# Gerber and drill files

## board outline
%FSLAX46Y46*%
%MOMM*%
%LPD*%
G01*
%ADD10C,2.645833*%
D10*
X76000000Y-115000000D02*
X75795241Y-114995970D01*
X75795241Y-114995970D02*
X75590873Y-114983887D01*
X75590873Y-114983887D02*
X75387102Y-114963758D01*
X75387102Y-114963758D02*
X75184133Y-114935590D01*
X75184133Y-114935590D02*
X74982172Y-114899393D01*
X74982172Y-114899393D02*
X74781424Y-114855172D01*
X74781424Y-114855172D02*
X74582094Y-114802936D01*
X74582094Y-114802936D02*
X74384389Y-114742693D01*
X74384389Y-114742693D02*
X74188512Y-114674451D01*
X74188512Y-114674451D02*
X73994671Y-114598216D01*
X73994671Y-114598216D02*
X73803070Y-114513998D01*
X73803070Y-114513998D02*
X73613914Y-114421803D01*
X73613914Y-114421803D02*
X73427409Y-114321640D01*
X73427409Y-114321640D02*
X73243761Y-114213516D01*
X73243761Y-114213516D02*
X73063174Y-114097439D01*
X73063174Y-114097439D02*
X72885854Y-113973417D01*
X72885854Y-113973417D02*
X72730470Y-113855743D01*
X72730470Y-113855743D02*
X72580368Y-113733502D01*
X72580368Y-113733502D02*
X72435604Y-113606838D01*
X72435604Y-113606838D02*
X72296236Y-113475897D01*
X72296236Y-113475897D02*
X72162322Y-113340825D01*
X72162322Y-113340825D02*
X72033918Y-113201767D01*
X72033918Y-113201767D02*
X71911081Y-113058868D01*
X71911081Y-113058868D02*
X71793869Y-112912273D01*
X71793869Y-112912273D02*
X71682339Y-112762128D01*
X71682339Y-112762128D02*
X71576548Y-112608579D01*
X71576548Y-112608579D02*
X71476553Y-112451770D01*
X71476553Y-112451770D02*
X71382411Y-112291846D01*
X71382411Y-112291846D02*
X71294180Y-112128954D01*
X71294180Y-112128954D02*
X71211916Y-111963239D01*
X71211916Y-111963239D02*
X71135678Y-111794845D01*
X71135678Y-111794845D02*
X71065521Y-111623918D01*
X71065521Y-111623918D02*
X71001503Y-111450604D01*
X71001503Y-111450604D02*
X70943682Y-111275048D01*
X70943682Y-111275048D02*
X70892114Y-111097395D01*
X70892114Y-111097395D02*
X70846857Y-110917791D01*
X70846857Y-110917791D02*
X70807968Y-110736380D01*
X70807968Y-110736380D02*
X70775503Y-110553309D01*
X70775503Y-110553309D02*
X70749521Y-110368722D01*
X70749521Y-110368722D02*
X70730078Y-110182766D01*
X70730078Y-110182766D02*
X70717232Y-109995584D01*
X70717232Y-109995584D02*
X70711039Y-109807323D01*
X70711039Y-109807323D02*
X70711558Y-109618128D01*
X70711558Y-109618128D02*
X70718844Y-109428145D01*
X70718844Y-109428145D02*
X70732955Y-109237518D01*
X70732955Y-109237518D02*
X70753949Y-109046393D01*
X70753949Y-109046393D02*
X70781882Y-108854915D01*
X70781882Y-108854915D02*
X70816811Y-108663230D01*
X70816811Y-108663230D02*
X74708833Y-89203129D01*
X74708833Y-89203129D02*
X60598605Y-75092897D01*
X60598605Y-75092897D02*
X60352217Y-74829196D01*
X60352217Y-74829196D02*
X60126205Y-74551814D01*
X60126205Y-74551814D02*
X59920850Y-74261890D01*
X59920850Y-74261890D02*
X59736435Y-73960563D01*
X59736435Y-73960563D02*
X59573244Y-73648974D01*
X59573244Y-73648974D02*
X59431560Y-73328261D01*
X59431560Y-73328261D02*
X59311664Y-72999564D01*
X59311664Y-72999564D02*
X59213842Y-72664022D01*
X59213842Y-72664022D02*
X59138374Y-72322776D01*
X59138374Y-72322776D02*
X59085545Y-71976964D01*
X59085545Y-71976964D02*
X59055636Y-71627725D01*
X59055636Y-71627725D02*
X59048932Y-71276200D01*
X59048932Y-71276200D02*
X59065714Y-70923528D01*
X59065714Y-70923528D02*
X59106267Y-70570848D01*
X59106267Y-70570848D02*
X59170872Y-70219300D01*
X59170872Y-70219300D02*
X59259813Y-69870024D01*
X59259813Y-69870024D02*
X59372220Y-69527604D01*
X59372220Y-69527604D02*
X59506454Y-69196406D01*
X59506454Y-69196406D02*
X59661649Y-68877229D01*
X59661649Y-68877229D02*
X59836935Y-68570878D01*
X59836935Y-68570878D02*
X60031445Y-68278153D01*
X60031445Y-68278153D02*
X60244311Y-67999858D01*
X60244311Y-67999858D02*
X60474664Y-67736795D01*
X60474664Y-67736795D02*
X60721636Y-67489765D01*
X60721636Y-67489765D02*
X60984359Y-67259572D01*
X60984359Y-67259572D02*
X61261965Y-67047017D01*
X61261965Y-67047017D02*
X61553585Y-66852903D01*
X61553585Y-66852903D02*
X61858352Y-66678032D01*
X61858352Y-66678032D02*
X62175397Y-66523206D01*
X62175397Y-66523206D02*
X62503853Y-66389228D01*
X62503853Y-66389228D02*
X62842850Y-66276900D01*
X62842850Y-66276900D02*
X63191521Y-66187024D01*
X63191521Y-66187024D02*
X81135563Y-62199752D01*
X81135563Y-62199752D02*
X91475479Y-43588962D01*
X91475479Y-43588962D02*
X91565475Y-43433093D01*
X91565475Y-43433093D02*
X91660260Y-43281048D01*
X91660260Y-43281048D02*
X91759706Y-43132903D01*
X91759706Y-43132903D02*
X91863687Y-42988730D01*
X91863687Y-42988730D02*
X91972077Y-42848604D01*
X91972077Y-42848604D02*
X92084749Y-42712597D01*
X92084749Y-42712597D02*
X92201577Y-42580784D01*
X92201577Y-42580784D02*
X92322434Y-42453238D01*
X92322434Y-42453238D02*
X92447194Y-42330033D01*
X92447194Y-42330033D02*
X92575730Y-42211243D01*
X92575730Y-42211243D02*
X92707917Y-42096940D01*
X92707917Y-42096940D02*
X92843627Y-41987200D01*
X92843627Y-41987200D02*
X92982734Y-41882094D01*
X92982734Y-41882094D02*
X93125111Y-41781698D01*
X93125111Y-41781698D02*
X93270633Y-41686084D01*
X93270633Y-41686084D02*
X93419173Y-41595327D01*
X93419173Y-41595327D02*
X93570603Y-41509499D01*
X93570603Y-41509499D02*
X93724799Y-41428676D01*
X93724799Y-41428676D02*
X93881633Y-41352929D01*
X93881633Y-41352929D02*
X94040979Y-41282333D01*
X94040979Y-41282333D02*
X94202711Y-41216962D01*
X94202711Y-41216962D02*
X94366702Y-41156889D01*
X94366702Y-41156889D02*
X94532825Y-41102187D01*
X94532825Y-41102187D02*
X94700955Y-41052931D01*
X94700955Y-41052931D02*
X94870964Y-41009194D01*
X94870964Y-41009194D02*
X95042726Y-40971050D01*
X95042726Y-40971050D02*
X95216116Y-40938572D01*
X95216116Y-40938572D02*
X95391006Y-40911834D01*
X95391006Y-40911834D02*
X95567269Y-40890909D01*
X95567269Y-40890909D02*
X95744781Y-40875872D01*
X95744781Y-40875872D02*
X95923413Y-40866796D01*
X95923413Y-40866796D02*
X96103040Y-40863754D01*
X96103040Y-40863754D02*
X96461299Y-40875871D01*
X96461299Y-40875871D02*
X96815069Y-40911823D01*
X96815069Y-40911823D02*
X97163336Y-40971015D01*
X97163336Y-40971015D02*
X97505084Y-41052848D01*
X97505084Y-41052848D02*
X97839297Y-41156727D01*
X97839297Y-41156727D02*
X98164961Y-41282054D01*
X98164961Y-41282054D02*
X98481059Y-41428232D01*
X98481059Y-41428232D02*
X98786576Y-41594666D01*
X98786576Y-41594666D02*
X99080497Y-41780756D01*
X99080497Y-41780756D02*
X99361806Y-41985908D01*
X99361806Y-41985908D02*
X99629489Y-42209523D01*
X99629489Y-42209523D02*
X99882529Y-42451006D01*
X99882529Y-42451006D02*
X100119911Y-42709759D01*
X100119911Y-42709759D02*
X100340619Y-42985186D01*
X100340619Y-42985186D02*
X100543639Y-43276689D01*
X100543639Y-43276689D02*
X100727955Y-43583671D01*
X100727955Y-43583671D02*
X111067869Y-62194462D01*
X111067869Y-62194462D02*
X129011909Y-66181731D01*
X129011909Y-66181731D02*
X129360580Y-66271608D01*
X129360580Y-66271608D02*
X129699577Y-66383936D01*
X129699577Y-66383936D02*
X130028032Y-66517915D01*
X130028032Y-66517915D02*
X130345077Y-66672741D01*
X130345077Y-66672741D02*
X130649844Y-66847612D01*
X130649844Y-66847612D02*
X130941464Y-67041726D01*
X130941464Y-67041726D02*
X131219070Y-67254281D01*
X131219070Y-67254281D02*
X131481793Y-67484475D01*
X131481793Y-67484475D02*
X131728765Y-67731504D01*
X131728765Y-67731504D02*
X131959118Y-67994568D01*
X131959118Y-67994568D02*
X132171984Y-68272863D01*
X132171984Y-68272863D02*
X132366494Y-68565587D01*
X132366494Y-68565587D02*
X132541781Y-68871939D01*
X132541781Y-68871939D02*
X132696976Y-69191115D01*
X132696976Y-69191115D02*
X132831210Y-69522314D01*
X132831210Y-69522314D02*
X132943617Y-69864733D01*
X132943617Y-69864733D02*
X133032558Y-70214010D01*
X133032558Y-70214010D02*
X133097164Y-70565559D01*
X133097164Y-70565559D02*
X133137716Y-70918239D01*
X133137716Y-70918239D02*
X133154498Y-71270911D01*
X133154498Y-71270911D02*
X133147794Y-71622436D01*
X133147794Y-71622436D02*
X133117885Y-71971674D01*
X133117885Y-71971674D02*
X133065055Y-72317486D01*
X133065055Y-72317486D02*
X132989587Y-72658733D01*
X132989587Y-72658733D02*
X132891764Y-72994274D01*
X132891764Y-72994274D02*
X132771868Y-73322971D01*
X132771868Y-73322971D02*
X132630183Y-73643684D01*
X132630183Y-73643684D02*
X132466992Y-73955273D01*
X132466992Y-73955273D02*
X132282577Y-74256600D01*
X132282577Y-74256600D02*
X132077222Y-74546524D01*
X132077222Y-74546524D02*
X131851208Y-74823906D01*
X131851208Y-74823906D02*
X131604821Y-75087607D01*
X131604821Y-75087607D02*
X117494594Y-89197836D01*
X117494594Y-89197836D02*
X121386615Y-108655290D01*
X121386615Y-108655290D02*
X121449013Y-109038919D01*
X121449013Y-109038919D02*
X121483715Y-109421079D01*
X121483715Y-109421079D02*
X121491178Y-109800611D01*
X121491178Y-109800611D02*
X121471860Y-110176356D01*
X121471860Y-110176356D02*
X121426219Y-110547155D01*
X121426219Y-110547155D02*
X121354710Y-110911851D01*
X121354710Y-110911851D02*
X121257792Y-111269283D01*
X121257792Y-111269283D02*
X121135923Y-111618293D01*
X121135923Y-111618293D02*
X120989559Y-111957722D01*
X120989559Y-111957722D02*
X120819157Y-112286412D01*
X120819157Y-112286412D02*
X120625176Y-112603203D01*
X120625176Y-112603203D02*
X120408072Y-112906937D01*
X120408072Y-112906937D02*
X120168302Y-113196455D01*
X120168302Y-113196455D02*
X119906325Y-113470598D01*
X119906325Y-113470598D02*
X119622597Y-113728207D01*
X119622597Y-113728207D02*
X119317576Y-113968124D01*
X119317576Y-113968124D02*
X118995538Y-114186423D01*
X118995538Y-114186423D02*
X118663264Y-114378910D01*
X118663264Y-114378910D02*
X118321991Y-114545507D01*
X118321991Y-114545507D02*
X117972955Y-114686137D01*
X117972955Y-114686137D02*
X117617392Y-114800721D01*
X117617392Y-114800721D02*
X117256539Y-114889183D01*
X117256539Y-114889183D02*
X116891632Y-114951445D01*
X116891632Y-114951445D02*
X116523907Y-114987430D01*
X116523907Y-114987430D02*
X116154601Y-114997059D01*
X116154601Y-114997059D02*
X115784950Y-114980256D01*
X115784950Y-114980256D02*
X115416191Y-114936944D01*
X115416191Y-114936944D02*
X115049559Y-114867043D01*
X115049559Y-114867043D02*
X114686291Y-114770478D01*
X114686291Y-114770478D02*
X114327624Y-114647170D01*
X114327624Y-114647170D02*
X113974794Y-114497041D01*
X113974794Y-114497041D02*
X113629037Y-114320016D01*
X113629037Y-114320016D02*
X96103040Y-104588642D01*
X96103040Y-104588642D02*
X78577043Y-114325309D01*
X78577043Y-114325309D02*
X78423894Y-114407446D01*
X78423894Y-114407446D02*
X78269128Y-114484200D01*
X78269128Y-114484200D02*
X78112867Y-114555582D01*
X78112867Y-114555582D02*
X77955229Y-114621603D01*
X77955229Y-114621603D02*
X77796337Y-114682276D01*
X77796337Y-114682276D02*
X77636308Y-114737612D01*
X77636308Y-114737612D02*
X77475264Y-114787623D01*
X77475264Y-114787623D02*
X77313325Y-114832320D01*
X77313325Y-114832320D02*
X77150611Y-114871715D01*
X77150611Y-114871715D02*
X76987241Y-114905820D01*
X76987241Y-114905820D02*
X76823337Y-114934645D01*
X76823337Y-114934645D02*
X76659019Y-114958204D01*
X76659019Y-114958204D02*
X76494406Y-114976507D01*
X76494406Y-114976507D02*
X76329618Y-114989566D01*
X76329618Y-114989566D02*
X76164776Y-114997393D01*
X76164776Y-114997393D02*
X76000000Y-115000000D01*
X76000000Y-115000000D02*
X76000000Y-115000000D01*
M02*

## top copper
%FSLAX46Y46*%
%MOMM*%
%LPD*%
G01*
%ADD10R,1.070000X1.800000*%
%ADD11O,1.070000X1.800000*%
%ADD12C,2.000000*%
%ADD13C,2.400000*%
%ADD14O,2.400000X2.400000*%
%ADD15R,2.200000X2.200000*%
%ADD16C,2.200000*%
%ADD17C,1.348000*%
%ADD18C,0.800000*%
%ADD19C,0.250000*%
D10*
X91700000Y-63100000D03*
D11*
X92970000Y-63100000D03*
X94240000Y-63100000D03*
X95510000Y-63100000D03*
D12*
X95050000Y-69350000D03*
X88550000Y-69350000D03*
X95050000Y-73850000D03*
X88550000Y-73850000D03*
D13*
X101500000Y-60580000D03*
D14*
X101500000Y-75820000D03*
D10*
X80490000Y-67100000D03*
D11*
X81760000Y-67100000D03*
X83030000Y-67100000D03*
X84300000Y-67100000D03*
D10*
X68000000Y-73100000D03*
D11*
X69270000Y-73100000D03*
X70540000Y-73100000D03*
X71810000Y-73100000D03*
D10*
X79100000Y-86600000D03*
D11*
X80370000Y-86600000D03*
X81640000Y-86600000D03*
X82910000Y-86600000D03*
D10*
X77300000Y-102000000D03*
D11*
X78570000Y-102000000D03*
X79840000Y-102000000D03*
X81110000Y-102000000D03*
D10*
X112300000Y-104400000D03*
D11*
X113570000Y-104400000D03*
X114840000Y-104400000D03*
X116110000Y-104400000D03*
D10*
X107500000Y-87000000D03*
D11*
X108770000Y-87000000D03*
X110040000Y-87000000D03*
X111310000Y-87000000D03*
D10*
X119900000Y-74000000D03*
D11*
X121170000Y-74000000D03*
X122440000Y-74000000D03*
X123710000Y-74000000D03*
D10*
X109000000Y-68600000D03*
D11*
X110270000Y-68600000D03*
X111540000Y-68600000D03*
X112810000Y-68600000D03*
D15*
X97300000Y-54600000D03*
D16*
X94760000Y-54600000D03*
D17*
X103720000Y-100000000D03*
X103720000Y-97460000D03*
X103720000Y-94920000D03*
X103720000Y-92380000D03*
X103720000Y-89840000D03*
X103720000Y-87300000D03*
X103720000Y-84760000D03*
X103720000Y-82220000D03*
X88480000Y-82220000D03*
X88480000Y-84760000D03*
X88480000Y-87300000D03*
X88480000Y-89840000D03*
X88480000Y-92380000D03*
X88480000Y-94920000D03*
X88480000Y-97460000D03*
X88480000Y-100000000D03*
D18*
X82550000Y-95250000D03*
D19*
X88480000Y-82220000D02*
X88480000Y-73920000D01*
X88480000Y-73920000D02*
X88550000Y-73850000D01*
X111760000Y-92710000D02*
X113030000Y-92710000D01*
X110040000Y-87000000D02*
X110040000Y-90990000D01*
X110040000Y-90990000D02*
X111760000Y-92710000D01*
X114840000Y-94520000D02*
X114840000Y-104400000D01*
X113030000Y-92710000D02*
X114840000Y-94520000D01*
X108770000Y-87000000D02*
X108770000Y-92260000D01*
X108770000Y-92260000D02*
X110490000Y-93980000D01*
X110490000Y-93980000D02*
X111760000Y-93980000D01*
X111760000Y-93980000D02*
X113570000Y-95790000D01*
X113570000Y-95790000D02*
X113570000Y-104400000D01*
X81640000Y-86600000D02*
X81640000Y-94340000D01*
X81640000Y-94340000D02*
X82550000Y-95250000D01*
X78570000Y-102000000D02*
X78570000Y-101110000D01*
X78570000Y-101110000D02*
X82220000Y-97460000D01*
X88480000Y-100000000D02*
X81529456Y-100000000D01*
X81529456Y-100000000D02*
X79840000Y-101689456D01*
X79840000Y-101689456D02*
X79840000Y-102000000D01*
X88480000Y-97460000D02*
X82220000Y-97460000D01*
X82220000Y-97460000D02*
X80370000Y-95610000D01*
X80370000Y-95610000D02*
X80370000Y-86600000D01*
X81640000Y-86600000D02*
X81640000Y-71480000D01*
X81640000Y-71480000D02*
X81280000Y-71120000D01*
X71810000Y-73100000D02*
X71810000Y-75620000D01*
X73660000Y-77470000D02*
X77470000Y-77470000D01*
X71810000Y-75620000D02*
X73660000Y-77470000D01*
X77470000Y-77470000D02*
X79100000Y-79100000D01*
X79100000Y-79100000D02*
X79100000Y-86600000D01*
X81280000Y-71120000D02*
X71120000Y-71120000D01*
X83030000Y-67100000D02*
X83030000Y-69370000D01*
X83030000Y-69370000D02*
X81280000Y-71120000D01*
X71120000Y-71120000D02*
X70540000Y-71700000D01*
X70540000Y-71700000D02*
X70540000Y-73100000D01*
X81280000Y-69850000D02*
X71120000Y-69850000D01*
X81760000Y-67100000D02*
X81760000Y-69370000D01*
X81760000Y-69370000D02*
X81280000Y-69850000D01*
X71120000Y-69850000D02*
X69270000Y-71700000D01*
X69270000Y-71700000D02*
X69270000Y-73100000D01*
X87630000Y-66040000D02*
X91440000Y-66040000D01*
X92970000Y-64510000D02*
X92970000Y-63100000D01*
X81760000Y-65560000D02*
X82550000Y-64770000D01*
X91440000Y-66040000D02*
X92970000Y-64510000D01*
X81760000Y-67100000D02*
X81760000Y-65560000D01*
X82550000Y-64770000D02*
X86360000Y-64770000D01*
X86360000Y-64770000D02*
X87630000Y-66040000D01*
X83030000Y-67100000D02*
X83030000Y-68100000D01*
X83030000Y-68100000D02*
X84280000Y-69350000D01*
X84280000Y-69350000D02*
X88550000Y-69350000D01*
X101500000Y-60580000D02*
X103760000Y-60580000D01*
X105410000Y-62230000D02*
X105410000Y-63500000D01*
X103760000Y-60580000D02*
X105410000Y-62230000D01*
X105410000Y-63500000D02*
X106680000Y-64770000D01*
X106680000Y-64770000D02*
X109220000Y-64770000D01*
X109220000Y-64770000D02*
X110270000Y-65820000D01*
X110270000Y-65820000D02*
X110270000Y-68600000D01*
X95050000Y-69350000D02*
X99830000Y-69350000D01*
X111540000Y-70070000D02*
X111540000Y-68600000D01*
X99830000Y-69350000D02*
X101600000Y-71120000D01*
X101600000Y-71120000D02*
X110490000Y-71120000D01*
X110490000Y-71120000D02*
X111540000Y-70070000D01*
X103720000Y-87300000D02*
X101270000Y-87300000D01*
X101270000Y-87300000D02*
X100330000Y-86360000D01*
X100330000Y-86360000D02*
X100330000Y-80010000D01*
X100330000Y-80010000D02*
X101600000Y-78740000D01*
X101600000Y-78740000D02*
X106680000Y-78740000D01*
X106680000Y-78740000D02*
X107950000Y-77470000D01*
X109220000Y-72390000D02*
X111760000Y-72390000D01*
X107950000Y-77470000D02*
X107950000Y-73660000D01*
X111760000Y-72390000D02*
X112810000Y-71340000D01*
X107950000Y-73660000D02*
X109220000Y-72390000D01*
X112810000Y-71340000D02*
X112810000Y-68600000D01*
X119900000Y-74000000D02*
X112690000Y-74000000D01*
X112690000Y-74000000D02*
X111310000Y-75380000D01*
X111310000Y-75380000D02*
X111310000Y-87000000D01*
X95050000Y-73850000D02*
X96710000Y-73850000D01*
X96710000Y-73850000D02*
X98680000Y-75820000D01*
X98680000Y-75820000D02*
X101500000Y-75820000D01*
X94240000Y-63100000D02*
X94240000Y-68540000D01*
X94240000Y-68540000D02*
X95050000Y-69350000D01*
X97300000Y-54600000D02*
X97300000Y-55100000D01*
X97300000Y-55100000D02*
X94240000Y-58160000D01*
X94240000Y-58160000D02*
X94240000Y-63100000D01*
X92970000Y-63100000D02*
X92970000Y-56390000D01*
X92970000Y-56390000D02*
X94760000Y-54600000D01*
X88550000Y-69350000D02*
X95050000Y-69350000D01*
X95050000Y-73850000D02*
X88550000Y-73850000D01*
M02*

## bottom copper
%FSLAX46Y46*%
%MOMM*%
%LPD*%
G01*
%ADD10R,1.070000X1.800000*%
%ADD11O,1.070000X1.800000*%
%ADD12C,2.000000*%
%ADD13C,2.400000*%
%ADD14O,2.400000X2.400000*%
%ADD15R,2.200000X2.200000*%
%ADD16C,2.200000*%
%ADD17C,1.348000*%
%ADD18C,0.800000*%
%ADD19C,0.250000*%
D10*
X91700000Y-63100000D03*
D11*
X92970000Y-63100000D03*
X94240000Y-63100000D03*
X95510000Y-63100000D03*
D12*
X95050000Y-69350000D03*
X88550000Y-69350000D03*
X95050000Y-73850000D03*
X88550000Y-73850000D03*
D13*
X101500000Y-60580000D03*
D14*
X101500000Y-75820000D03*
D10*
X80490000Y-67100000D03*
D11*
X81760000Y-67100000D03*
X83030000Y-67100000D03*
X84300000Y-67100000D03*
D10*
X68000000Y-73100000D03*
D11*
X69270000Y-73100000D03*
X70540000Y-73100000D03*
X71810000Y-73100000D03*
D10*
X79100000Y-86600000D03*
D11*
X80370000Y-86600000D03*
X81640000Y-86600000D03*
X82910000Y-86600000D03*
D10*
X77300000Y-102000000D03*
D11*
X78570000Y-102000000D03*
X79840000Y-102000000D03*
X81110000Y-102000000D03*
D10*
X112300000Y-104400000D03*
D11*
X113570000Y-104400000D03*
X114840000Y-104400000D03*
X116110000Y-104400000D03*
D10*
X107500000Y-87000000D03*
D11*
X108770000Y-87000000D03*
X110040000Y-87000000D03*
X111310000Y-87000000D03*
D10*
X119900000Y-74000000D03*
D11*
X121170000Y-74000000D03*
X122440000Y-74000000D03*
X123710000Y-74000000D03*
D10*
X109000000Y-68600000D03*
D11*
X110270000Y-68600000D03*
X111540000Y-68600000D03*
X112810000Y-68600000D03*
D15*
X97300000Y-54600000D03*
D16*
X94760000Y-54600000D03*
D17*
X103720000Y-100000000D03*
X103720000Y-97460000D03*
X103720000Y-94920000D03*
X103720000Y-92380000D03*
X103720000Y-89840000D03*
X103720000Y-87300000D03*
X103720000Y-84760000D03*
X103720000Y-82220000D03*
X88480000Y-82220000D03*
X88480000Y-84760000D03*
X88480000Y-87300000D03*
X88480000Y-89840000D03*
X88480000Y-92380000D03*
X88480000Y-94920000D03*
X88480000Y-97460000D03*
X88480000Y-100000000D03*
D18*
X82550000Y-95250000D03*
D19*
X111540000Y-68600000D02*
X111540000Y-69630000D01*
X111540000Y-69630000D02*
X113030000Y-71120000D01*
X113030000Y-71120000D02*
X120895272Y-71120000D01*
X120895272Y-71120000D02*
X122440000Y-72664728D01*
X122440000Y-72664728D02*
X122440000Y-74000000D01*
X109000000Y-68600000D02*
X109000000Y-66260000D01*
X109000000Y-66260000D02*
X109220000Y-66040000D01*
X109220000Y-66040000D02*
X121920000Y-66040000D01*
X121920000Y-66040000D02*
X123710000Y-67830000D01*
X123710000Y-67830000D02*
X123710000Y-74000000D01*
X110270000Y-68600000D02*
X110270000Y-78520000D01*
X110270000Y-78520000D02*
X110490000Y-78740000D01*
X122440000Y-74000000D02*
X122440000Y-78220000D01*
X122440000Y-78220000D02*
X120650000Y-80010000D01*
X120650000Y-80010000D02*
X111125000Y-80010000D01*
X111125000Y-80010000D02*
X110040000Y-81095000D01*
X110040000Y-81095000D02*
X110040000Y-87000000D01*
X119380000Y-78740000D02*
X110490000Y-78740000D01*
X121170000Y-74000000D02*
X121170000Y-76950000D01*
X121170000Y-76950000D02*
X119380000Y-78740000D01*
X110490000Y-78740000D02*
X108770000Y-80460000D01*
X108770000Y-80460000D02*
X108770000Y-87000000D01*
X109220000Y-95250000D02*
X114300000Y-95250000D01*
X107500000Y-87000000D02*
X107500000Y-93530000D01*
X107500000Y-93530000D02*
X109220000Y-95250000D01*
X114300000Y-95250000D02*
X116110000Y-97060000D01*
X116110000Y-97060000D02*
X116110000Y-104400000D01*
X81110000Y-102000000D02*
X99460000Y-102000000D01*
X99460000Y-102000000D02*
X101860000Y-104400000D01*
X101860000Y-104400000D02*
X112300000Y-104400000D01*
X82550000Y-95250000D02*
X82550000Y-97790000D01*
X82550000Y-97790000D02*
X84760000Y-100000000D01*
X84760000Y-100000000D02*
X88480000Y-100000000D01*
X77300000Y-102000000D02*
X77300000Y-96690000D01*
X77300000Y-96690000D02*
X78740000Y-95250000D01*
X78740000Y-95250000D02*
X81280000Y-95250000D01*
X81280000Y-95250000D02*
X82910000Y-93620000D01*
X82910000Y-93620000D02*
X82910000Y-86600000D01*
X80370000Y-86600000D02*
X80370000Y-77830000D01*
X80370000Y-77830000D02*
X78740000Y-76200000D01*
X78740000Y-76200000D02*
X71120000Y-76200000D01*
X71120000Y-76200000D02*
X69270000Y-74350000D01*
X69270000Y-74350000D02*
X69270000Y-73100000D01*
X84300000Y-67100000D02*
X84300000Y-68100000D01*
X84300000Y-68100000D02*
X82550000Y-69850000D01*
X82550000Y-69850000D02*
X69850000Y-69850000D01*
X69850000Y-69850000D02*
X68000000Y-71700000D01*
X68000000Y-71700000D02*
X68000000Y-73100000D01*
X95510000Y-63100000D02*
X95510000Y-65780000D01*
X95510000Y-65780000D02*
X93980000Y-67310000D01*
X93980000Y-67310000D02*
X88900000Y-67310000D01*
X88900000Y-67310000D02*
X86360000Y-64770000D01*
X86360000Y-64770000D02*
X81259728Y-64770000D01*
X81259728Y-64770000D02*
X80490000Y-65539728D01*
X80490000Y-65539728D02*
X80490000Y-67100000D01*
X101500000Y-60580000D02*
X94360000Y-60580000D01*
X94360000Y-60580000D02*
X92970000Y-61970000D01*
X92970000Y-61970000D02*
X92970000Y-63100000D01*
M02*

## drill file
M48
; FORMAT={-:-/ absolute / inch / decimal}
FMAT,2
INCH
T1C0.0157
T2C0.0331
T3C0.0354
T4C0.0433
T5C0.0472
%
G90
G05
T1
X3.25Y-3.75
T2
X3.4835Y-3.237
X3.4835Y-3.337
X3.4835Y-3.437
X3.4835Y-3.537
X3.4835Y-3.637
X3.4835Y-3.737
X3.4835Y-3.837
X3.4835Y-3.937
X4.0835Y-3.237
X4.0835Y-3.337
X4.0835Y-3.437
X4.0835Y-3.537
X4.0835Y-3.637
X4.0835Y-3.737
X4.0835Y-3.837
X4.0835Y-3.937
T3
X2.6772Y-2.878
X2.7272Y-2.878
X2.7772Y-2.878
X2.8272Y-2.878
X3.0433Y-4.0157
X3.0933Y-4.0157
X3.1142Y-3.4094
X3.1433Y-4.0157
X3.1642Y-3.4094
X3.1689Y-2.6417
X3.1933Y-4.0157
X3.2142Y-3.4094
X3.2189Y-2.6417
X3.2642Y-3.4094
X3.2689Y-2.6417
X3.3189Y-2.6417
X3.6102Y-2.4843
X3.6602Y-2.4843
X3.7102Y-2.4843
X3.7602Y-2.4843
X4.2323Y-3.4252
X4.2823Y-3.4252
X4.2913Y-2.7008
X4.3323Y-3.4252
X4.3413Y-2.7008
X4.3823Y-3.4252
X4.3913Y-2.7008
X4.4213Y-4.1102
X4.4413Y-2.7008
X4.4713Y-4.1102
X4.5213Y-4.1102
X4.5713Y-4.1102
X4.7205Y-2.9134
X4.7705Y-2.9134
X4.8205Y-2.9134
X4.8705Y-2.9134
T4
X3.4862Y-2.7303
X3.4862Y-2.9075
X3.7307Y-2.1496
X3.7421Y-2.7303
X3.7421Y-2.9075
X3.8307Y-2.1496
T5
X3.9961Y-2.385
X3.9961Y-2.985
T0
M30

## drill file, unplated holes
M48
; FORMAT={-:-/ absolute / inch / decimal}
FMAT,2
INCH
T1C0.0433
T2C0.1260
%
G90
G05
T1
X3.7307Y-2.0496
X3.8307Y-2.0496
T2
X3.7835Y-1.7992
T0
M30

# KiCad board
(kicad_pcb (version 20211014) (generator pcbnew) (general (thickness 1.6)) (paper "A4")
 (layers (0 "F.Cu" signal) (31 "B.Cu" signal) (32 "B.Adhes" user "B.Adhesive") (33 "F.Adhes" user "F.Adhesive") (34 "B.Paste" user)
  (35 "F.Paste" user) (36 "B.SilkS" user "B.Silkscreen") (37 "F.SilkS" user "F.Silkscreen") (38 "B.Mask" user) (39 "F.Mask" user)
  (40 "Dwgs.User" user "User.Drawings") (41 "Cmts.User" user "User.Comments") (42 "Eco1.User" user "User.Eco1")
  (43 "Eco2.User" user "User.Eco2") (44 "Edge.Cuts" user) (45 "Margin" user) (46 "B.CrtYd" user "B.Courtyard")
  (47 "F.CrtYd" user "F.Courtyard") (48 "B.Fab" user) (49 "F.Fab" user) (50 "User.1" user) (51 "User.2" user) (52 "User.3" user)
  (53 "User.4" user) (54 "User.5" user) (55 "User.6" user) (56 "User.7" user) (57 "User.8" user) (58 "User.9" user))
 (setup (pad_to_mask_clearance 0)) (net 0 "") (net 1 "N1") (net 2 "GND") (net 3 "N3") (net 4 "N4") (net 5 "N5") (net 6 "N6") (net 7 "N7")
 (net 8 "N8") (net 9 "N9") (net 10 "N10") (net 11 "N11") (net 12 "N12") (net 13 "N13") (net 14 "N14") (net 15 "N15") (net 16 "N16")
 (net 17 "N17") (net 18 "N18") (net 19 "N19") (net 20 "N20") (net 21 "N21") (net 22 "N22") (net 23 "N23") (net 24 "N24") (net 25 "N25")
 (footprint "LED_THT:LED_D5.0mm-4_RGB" (layer "F.Cu") (at 77.3 102)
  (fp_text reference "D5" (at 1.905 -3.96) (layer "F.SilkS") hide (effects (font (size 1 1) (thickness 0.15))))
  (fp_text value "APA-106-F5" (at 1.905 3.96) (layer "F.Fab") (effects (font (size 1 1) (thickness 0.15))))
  (pad "1" thru_hole rect (at 0 0) (size 1.07 1.8) (drill 0.9) (layers *.Cu *.Mask) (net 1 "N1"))
  (pad "2" thru_hole oval (at 1.27 0) (size 1.07 1.8) (drill 0.9) (layers *.Cu *.Mask) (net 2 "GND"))
  (pad "3" thru_hole oval (at 2.54 0) (size 1.07 1.8) (drill 0.9) (layers *.Cu *.Mask) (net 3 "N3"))
  (pad "4" thru_hole oval (at 3.81 0) (size 1.07 1.8) (drill 0.9) (layers *.Cu *.Mask) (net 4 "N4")))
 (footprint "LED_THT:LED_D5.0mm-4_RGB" (layer "F.Cu") (at 119.9 74)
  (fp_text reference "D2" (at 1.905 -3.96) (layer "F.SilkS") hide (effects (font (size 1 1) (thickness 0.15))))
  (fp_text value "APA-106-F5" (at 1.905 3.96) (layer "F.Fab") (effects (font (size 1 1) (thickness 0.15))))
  (pad "1" thru_hole rect (at 0 0) (size 1.07 1.8) (drill 0.9) (layers *.Cu *.Mask) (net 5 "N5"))
  (pad "2" thru_hole oval (at 1.27 0) (size 1.07 1.8) (drill 0.9) (layers *.Cu *.Mask) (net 2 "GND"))
  (pad "3" thru_hole oval (at 2.54 0) (size 1.07 1.8) (drill 0.9) (layers *.Cu *.Mask) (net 3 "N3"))
  (pad "4" thru_hole oval (at 3.81 0) (size 1.07 1.8) (drill 0.9) (layers *.Cu *.Mask) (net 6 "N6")))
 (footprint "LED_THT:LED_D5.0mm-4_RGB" (layer "F.Cu") (at 80.49 67.1)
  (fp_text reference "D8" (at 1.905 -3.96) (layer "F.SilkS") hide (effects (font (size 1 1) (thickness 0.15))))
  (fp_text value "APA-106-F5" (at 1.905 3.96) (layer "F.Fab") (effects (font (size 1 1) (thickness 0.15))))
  (pad "1" thru_hole rect (at 0 0) (size 1.07 1.8) (drill 0.9) (layers *.Cu *.Mask) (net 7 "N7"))
  (pad "2" thru_hole oval (at 1.27 0) (size 1.07 1.8) (drill 0.9) (layers *.Cu *.Mask) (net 2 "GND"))
  (pad "3" thru_hole oval (at 2.54 0) (size 1.07 1.8) (drill 0.9) (layers *.Cu *.Mask) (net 3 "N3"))
  (pad "4" thru_hole oval (at 3.81 0) (size 1.07 1.8) (drill 0.9) (layers *.Cu *.Mask) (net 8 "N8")))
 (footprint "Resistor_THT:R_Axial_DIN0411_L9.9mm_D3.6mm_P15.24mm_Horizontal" (layer "F.Cu") (at 101.5 60.58 -90)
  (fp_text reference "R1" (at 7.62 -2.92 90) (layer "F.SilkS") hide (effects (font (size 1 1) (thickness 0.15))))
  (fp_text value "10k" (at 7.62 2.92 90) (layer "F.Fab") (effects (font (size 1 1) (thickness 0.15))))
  (pad "1" thru_hole circle (at 0 0 270) (size 2.4 2.4) (drill 1.2) (layers *.Cu *.Mask) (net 2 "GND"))
  (pad "2" thru_hole oval (at 15.24 0 270) (size 2.4 2.4) (drill 1.2) (layers *.Cu *.Mask) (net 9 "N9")))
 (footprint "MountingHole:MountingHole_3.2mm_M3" (layer "F.Cu") (at 96.1 45.7)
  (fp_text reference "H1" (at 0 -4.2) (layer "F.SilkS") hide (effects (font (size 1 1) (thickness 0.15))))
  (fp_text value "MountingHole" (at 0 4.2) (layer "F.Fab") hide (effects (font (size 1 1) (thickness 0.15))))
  (pad "" np_thru_hole circle (at 0 0) (size 3.2 3.2) (drill 3.2) (layers *.Cu *.Mask)))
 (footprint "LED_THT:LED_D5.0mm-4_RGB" (layer "F.Cu") (at 91.7 63.1)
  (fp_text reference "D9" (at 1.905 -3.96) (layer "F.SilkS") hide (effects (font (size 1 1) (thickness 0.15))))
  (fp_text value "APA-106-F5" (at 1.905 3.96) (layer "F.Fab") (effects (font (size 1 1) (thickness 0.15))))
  (pad "1" thru_hole rect (at 0 0) (size 1.07 1.8) (drill 0.9) (layers *.Cu *.Mask) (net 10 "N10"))
  (pad "2" thru_hole oval (at 1.27 0) (size 1.07 1.8) (drill 0.9) (layers *.Cu *.Mask) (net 2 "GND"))
  (pad "3" thru_hole oval (at 2.54 0) (size 1.07 1.8) (drill 0.9) (layers *.Cu *.Mask) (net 3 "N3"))
  (pad "4" thru_hole oval (at 3.81 0) (size 1.07 1.8) (drill 0.9) (layers *.Cu *.Mask) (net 7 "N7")))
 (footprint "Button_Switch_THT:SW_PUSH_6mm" (layer "F.Cu") (at 88.55 69.35)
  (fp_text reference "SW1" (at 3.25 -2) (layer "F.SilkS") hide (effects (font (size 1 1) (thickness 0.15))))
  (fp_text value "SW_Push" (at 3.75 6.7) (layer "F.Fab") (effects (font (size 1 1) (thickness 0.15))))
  (pad "1" thru_hole circle (at 0 0 90) (size 2 2) (drill 1.1) (layers *.Cu *.Mask) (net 3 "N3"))
  (pad "1" thru_hole circle (at 6.5 0 90) (size 2 2) (drill 1.1) (layers *.Cu *.Mask) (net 3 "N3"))
  (pad "2" thru_hole circle (at 6.5 4.5 90) (size 2 2) (drill 1.1) (layers *.Cu *.Mask) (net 9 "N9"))
  (pad "2" thru_hole circle (at 0 4.5 90) (size 2 2) (drill 1.1) (layers *.Cu *.Mask) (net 9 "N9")))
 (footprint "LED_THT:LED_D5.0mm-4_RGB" (layer "F.Cu") (at 79.1 86.6)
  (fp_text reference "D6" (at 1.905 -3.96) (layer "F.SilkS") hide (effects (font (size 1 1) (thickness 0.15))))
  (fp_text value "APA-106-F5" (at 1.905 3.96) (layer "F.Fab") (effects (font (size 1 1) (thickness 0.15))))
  (pad "1" thru_hole rect (at 0 0) (size 1.07 1.8) (drill 0.9) (layers *.Cu *.Mask) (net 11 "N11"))
  (pad "2" thru_hole oval (at 1.27 0) (size 1.07 1.8) (drill 0.9) (layers *.Cu *.Mask) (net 2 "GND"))
  (pad "3" thru_hole oval (at 2.54 0) (size 1.07 1.8) (drill 0.9) (layers *.Cu *.Mask) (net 3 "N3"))
  (pad "4" thru_hole oval (at 3.81 0) (size 1.07 1.8) (drill 0.9) (layers *.Cu *.Mask) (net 1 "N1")))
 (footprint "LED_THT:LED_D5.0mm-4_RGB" (layer "F.Cu") (at 112.3 104.4)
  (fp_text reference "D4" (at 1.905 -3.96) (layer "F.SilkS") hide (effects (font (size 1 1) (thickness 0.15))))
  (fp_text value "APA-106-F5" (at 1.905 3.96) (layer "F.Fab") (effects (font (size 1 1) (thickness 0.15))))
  (pad "1" thru_hole rect (at 0 0) (size 1.07 1.8) (drill 0.9) (layers *.Cu *.Mask) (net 4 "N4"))
  (pad "2" thru_hole oval (at 1.27 0) (size 1.07 1.8) (drill 0.9) (layers *.Cu *.Mask) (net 2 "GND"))
  (pad "3" thru_hole oval (at 2.54 0) (size 1.07 1.8) (drill 0.9) (layers *.Cu *.Mask) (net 3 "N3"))
  (pad "4" thru_hole oval (at 3.81 0) (size 1.07 1.8) (drill 0.9) (layers *.Cu *.Mask) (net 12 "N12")))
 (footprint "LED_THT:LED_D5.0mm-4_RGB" (layer "F.Cu") (at 109 68.6)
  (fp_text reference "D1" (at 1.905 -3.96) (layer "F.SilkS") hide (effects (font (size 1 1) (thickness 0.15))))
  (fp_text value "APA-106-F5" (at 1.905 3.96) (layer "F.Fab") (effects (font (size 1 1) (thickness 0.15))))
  (pad "1" thru_hole rect (at 0 0) (size 1.07 1.8) (drill 0.9) (layers *.Cu *.Mask) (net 6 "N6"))
  (pad "2" thru_hole oval (at 1.27 0) (size 1.07 1.8) (drill 0.9) (layers *.Cu *.Mask) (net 2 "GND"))
  (pad "3" thru_hole oval (at 2.54 0) (size 1.07 1.8) (drill 0.9) (layers *.Cu *.Mask) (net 3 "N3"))
  (pad "4" thru_hole oval (at 3.81 0) (size 1.07 1.8) (drill 0.9) (layers *.Cu *.Mask) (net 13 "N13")))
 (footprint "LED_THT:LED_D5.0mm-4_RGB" (layer "F.Cu") (at 107.5 87)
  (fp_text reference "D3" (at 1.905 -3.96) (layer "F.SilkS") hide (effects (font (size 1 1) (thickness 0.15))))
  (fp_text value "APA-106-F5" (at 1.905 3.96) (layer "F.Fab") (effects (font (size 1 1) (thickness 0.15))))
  (pad "1" thru_hole rect (at 0 0) (size 1.07 1.8) (drill 0.9) (layers *.Cu *.Mask) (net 12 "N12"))
  (pad "2" thru_hole oval (at 1.27 0) (size 1.07 1.8) (drill 0.9) (layers *.Cu *.Mask) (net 2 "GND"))
  (pad "3" thru_hole oval (at 2.54 0) (size 1.07 1.8) (drill 0.9) (layers *.Cu *.Mask) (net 3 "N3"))
  (pad "4" thru_hole oval (at 3.81 0) (size 1.07 1.8) (drill 0.9) (layers *.Cu *.Mask) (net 5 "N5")))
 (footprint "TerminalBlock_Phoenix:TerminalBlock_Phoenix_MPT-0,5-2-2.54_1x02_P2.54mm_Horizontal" (layer "F.Cu") (at 97.3 54.6 180)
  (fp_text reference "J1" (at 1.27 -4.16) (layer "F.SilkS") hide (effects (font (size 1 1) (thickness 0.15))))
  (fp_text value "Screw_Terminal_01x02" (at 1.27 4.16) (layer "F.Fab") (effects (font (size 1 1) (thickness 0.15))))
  (pad "" np_thru_hole circle (at 0 2.54 180) (size 1.1 1.1) (drill 1.1) (layers *.Cu *.Mask))
  (pad "" np_thru_hole circle (at 2.54 2.54 180) (size 1.1 1.1) (drill 1.1) (layers *.Cu *.Mask))
  (pad "1" thru_hole rect (at 0 0 180) (size 2.2 2.2) (drill 1.1) (layers *.Cu *.Mask) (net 3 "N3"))
  (pad "2" thru_hole circle (at 2.54 0 180) (size 2.2 2.2) (drill 1.1) (layers *.Cu *.Mask) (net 2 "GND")))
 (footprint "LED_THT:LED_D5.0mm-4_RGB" (layer "F.Cu") (at 68 73.1)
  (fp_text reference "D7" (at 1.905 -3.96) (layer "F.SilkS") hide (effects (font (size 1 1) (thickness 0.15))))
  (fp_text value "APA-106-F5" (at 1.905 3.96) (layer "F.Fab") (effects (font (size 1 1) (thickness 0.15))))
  (pad "1" thru_hole rect (at 0 0) (size 1.07 1.8) (drill 0.9) (layers *.Cu *.Mask) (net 8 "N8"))
  (pad "2" thru_hole oval (at 1.27 0) (size 1.07 1.8) (drill 0.9) (layers *.Cu *.Mask) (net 2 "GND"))
  (pad "3" thru_hole oval (at 2.54 0) (size 1.07 1.8) (drill 0.9) (layers *.Cu *.Mask) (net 3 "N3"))
  (pad "4" thru_hole oval (at 3.81 0) (size 1.07 1.8) (drill 0.9) (layers *.Cu *.Mask) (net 11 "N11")))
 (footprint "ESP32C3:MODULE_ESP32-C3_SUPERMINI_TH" (layer "F.Cu") (at 96.1 90.1 180)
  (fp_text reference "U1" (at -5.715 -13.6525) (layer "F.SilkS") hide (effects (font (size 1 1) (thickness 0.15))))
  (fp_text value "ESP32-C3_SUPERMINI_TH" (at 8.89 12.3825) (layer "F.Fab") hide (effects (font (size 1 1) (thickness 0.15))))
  (pad "0" thru_hole circle locked (at 7.62 7.88 180) (size 1.348 1.348) (drill 0.84) (layers *.Cu *.Mask) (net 9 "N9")
   (solder_mask_margin 0.102))
  (pad "1" thru_hole circle locked (at 7.62 5.34 180) (size 1.348 1.348) (drill 0.84) (layers *.Cu *.Mask) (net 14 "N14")
   (solder_mask_margin 0.102))
  (pad "2" thru_hole circle locked (at 7.62 2.8 180) (size 1.348 1.348) (drill 0.84) (layers *.Cu *.Mask) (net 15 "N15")
   (solder_mask_margin 0.102))
  (pad "3" thru_hole circle locked (at 7.62 0.26 180) (size 1.348 1.348) (drill 0.84) (layers *.Cu *.Mask) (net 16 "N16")
   (solder_mask_margin 0.102))
  (pad "3.3" thru_hole circle locked (at 7.62 -4.82 180) (size 1.348 1.348) (drill 0.84) (layers *.Cu *.Mask) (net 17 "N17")
   (solder_mask_margin 0.102))
  (pad "4" thru_hole circle locked (at 7.62 -2.28 180) (size 1.348 1.348) (drill 0.84) (layers *.Cu *.Mask) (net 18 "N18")
   (solder_mask_margin 0.102))
  (pad "5" thru_hole circle locked (at -7.62 -9.9 180) (size 1.348 1.348) (drill 0.84) (layers *.Cu *.Mask) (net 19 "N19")
   (solder_mask_margin 0.102))
  (pad "5V" thru_hole circle locked (at 7.62 -9.9 180) (size 1.348 1.348) (drill 0.84) (layers *.Cu *.Mask) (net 3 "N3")
   (solder_mask_margin 0.102))
  (pad "6" thru_hole circle locked (at -7.62 -7.36 180) (size 1.348 1.348) (drill 0.84) (layers *.Cu *.Mask) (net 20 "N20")
   (solder_mask_margin 0.102))
  (pad "7" thru_hole circle locked (at -7.62 -4.82 180) (size 1.348 1.348) (drill 0.84) (layers *.Cu *.Mask) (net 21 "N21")
   (solder_mask_margin 0.102))
  (pad "8" thru_hole circle locked (at -7.62 -2.28 180) (size 1.348 1.348) (drill 0.84) (layers *.Cu *.Mask) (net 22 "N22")
   (solder_mask_margin 0.102))
  (pad "9" thru_hole circle locked (at -7.62 0.26 180) (size 1.348 1.348) (drill 0.84) (layers *.Cu *.Mask) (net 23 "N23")
   (solder_mask_margin 0.102))
  (pad "10" thru_hole circle locked (at -7.62 2.8 180) (size 1.348 1.348) (drill 0.84) (layers *.Cu *.Mask) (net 13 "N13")
   (solder_mask_margin 0.102))
  (pad "20" thru_hole circle locked (at -7.62 5.34 180) (size 1.348 1.348) (drill 0.84) (layers *.Cu *.Mask) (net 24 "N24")
   (solder_mask_margin 0.102))
  (pad "21" thru_hole circle locked (at -7.62 7.88 180) (size 1.348 1.348) (drill 0.84) (layers *.Cu *.Mask) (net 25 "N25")
   (solder_mask_margin 0.102))
  (pad "G" thru_hole circle locked (at 7.62 -7.36 180) (size 1.348 1.348) (drill 0.84) (layers *.Cu *.Mask) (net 2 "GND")
   (solder_mask_margin 0.102)))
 (gr_poly
  (pts (xy 76 115) (xy 75.795241 114.99597) (xy 75.590873 114.983887) (xy 75.387102 114.963758) (xy 75.184133 114.93559)
   (xy 74.982172 114.899393) (xy 74.781424 114.855172) (xy 74.582094 114.802936) (xy 74.384389 114.742693) (xy 74.188512 114.674451)
   (xy 73.994671 114.598216) (xy 73.80307 114.513998) (xy 73.613914 114.421803) (xy 73.427409 114.32164) (xy 73.243761 114.213516)
   (xy 73.063174 114.097439) (xy 72.885854 113.973417) (xy 72.73047 113.855743) (xy 72.580368 113.733502) (xy 72.435604 113.606838)
   (xy 72.296236 113.475897) (xy 72.162322 113.340825) (xy 72.033918 113.201767) (xy 71.911081 113.058868) (xy 71.793869 112.912273)
   (xy 71.682339 112.762128) (xy 71.576548 112.608579) (xy 71.476553 112.45177) (xy 71.382411 112.291846) (xy 71.29418 112.128954)
   (xy 71.211916 111.963239) (xy 71.135678 111.794845) (xy 71.065521 111.623918) (xy 71.001503 111.450604) (xy 70.943682 111.275048)
   (xy 70.892114 111.097395) (xy 70.846857 110.917791) (xy 70.807968 110.73638) (xy 70.775503 110.553309) (xy 70.749521 110.368722)
   (xy 70.730078 110.182766) (xy 70.717232 109.995584) (xy 70.711039 109.807323) (xy 70.711558 109.618128) (xy 70.718844 109.428145)
   (xy 70.732955 109.237518) (xy 70.753949 109.046393) (xy 70.781882 108.854915) (xy 70.816811 108.66323) (xy 74.708833 89.203129)
   (xy 60.598605 75.092897) (xy 60.352217 74.829196) (xy 60.126205 74.551814) (xy 59.92085 74.26189) (xy 59.736435 73.960563)
   (xy 59.573244 73.648974) (xy 59.43156 73.328261) (xy 59.311664 72.999564) (xy 59.213842 72.664022) (xy 59.138374 72.322776)
   (xy 59.085545 71.976964) (xy 59.055636 71.627725) (xy 59.048932 71.2762) (xy 59.065714 70.923528) (xy 59.106267 70.570848)
   (xy 59.170872 70.2193) (xy 59.259813 69.870024) (xy 59.37222 69.527604) (xy 59.506454 69.196406) (xy 59.661649 68.877229)
   (xy 59.836935 68.570878) (xy 60.031445 68.278153) (xy 60.244311 67.999858) (xy 60.474664 67.736795) (xy 60.721636 67.489765)
   (xy 60.984359 67.259572) (xy 61.261965 67.047017) (xy 61.553585 66.852903) (xy 61.858352 66.678032) (xy 62.175397 66.523206)
   (xy 62.503853 66.389228) (xy 62.84285 66.2769) (xy 63.191521 66.187024) (xy 81.135563 62.199752) (xy 91.475479 43.588962)
   (xy 91.565475 43.433093) (xy 91.66026 43.281048) (xy 91.759706 43.132903) (xy 91.863687 42.98873) (xy 91.972077 42.848604)
   (xy 92.084749 42.712597) (xy 92.201577 42.580784) (xy 92.322434 42.453238) (xy 92.447194 42.330033) (xy 92.57573 42.211243)
   (xy 92.707917 42.09694) (xy 92.843627 41.9872) (xy 92.982734 41.882094) (xy 93.125111 41.781698) (xy 93.270633 41.686084)
   (xy 93.419173 41.595327) (xy 93.570603 41.509499) (xy 93.724799 41.428676) (xy 93.881633 41.352929) (xy 94.040979 41.282333)
   (xy 94.202711 41.216962) (xy 94.366702 41.156889) (xy 94.532825 41.102187) (xy 94.700955 41.052931) (xy 94.870964 41.009194)
   (xy 95.042726 40.97105) (xy 95.216116 40.938572) (xy 95.391006 40.911834) (xy 95.567269 40.890909) (xy 95.744781 40.875872)
   (xy 95.923413 40.866796) (xy 96.10304 40.863754) (xy 96.461299 40.875871) (xy 96.815069 40.911823) (xy 97.163336 40.971015)
   (xy 97.505084 41.052848) (xy 97.839297 41.156727) (xy 98.164961 41.282054) (xy 98.481059 41.428232) (xy 98.786576 41.594666)
   (xy 99.080497 41.780756) (xy 99.361806 41.985908) (xy 99.629489 42.209523) (xy 99.882529 42.451006) (xy 100.119911 42.709759)
   (xy 100.340619 42.985186) (xy 100.543639 43.276689) (xy 100.727955 43.583671) (xy 111.067869 62.194462) (xy 129.011909 66.181731)
   (xy 129.36058 66.271608) (xy 129.699577 66.383936) (xy 130.028032 66.517915) (xy 130.345077 66.672741) (xy 130.649844 66.847612)
   (xy 130.941464 67.041726) (xy 131.21907 67.254281) (xy 131.481793 67.484475) (xy 131.728765 67.731504) (xy 131.959118 67.994568)
   (xy 132.171984 68.272863) (xy 132.366494 68.565587) (xy 132.541781 68.871939) (xy 132.696976 69.191115) (xy 132.83121 69.522314)
   (xy 132.943617 69.864733) (xy 133.032558 70.21401) (xy 133.097164 70.565559) (xy 133.137716 70.918239) (xy 133.154498 71.270911)
   (xy 133.147794 71.622436) (xy 133.117885 71.971674) (xy 133.065055 72.317486) (xy 132.989587 72.658733) (xy 132.891764 72.994274)
   (xy 132.771868 73.322971) (xy 132.630183 73.643684) (xy 132.466992 73.955273) (xy 132.282577 74.2566) (xy 132.077222 74.546524)
   (xy 131.851208 74.823906) (xy 131.604821 75.087607) (xy 117.494594 89.197836) (xy 121.386615 108.65529) (xy 121.449013 109.038919)
   (xy 121.483715 109.421079) (xy 121.491178 109.800611) (xy 121.47186 110.176356) (xy 121.426219 110.547155) (xy 121.35471 110.911851)
   (xy 121.257792 111.269283) (xy 121.135923 111.618293) (xy 120.989559 111.957722) (xy 120.819157 112.286412) (xy 120.625176 112.603203)
   (xy 120.408072 112.906937) (xy 120.168302 113.196455) (xy 119.906325 113.470598) (xy 119.622597 113.728207) (xy 119.317576 113.968124)
   (xy 118.995538 114.186423) (xy 118.663264 114.37891) (xy 118.321991 114.545507) (xy 117.972955 114.686137) (xy 117.617392 114.800721)
   (xy 117.256539 114.889183) (xy 116.891632 114.951445) (xy 116.523907 114.98743) (xy 116.154601 114.997059) (xy 115.78495 114.980256)
   (xy 115.416191 114.936944) (xy 115.049559 114.867043) (xy 114.686291 114.770478) (xy 114.327624 114.64717) (xy 113.974794 114.497041)
   (xy 113.629037 114.320016) (xy 96.10304 104.588642) (xy 78.577043 114.325309) (xy 78.423894 114.407446) (xy 78.269128 114.4842)
   (xy 78.112867 114.555582) (xy 77.955229 114.621603) (xy 77.796337 114.682276) (xy 77.636308 114.737612) (xy 77.475264 114.787623)
   (xy 77.313325 114.83232) (xy 77.150611 114.871715) (xy 76.987241 114.90582) (xy 76.823337 114.934645) (xy 76.659019 114.958204)
   (xy 76.494406 114.976507) (xy 76.329618 114.989566) (xy 76.164776 114.997393) (xy 76 115))
  (layer "Edge.Cuts") (width 2.645833) (fill none))
 (segment (start 109.22 66.04) (end 121.92 66.04) (width 0.25) (layer "B.Cu") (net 6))
 (segment (start 121.92 66.04) (end 123.71 67.83) (width 0.25) (layer "B.Cu") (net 6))
 (segment (start 123.71 67.83) (end 123.71 74) (width 0.25) (layer "B.Cu") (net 6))
 (segment (start 109 68.6) (end 109 66.26) (width 0.25) (layer "B.Cu") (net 6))
 (segment (start 109 66.26) (end 109.22 66.04) (width 0.25) (layer "B.Cu") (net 6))
 (segment (start 81.28 69.85) (end 71.12 69.85) (width 0.25) (layer "F.Cu") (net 2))
 (segment (start 86.36 64.77) (end 87.63 66.04) (width 0.25) (layer "F.Cu") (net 2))
 (segment (start 81.76 69.37) (end 81.28 69.85) (width 0.25) (layer "F.Cu") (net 2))
 (segment (start 82.55 64.77) (end 86.36 64.77) (width 0.25) (layer "F.Cu") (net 2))
 (segment (start 105.41 62.23) (end 105.41 63.5) (width 0.25) (layer "F.Cu") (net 2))
 (segment (start 92.97 63.1) (end 92.97 56.39) (width 0.25) (layer "F.Cu") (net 2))
 (segment (start 110.49 93.98) (end 111.76 93.98) (width 0.25) (layer "F.Cu") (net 2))
 (segment (start 92.97 64.51) (end 92.97 63.1) (width 0.25) (layer "F.Cu") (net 2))
 (segment (start 71.12 69.85) (end 69.27 71.7) (width 0.25) (layer "F.Cu") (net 2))
 (segment (start 78.57 101.11) (end 82.22 97.46) (width 0.25) (layer "F.Cu") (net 2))
 (segment (start 80.37 95.61) (end 80.37 86.6) (width 0.25) (layer "F.Cu") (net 2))
 (segment (start 92.97 56.39) (end 94.76 54.6) (width 0.25) (layer "F.Cu") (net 2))
 (segment (start 106.68 64.77) (end 109.22 64.77) (width 0.25) (layer "F.Cu") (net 2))
 (segment (start 103.76 60.58) (end 105.41 62.23) (width 0.25) (layer "F.Cu") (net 2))
 (segment (start 105.41 63.5) (end 106.68 64.77) (width 0.25) (layer "F.Cu") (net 2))
 (segment (start 81.76 67.1) (end 81.76 65.56) (width 0.25) (layer "F.Cu") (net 2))
 (segment (start 87.63 66.04) (end 91.44 66.04) (width 0.25) (layer "F.Cu") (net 2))
 (segment (start 69.27 71.7) (end 69.27 73.1) (width 0.25) (layer "F.Cu") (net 2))
 (segment (start 110.27 65.82) (end 110.27 68.6) (width 0.25) (layer "F.Cu") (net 2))
 (segment (start 88.48 97.46) (end 82.22 97.46) (width 0.25) (layer "F.Cu") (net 2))
 (segment (start 101.5 60.58) (end 103.76 60.58) (width 0.25) (layer "F.Cu") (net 2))
 (segment (start 91.44 66.04) (end 92.97 64.51) (width 0.25) (layer "F.Cu") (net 2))
 (segment (start 81.76 65.56) (end 82.55 64.77) (width 0.25) (layer "F.Cu") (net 2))
 (segment (start 109.22 64.77) (end 110.27 65.82) (width 0.25) (layer "F.Cu") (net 2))
 (segment (start 111.76 93.98) (end 113.57 95.79) (width 0.25) (layer "F.Cu") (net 2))
 (segment (start 108.77 92.26) (end 110.49 93.98) (width 0.25) (layer "F.Cu") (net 2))
 (segment (start 78.57 102) (end 78.57 101.11) (width 0.25) (layer "F.Cu") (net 2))
 (segment (start 113.57 95.79) (end 113.57 104.4) (width 0.25) (layer "F.Cu") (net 2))
 (segment (start 82.22 97.46) (end 80.37 95.61) (width 0.25) (layer "F.Cu") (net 2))
 (segment (start 108.77 87) (end 108.77 92.26) (width 0.25) (layer "F.Cu") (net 2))
 (segment (start 81.76 67.1) (end 81.76 69.37) (width 0.25) (layer "F.Cu") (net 2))
 (segment (start 121.17 74) (end 121.17 76.95) (width 0.25) (layer "B.Cu") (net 2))
 (segment (start 110.27 68.6) (end 110.27 78.52) (width 0.25) (layer "B.Cu") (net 2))
 (segment (start 80.37 77.83) (end 78.74 76.2) (width 0.25) (layer "B.Cu") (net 2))
 (segment (start 69.27 74.35) (end 69.27 73.1) (width 0.25) (layer "B.Cu") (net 2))
 (segment (start 121.17 76.95) (end 119.38 78.74) (width 0.25) (layer "B.Cu") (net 2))
 (segment (start 78.74 76.2) (end 71.12 76.2) (width 0.25) (layer "B.Cu") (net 2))
 (segment (start 80.37 86.6) (end 80.37 77.83) (width 0.25) (layer "B.Cu") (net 2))
 (segment (start 101.5 60.58) (end 94.36 60.58) (width 0.25) (layer "B.Cu") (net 2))
 (segment (start 110.49 78.74) (end 108.77 80.46) (width 0.25) (layer "B.Cu") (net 2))
 (segment (start 71.12 76.2) (end 69.27 74.35) (width 0.25) (layer "B.Cu") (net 2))
 (segment (start 108.77 80.46) (end 108.77 87) (width 0.25) (layer "B.Cu") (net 2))
 (segment (start 92.97 61.97) (end 92.97 63.1) (width 0.25) (layer "B.Cu") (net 2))
 (segment (start 110.27 78.52) (end 110.49 78.74) (width 0.25) (layer "B.Cu") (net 2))
 (segment (start 94.36 60.58) (end 92.97 61.97) (width 0.25) (layer "B.Cu") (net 2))
 (segment (start 119.38 78.74) (end 110.49 78.74) (width 0.25) (layer "B.Cu") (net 2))
 (segment (start 101.6 71.12) (end 110.49 71.12) (width 0.25) (layer "F.Cu") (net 3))
 (segment (start 110.04 87) (end 110.04 90.99) (width 0.25) (layer "F.Cu") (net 3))
 (segment (start 81.64 86.6) (end 81.64 94.34) (width 0.25) (layer "F.Cu") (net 3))
 (segment (start 114.84 94.52) (end 114.84 104.4) (width 0.25) (layer "F.Cu") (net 3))
 (segment (start 88.55 69.35) (end 95.05 69.35) (width 0.25) (layer "F.Cu") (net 3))
 (segment (start 81.64 71.48) (end 81.28 71.12) (width 0.25) (layer "F.Cu") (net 3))
 (segment (start 97.3 54.6) (end 97.3 55.1) (width 0.25) (layer "F.Cu") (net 3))
 (segment (start 113.03 92.71) (end 114.84 94.52) (width 0.25) (layer "F.Cu") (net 3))
 (segment (start 83.03 67.1) (end 83.03 68.1) (width 0.25) (layer "F.Cu") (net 3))
 (segment (start 83.03 69.37) (end 81.28 71.12) (width 0.25) (layer "F.Cu") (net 3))
 (segment (start 70.54 71.7) (end 70.54 73.1) (width 0.25) (layer "F.Cu") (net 3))
 (segment (start 81.529456 100) (end 79.84 101.689456) (width 0.25) (layer "F.Cu") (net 3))
 (segment (start 79.84 101.689456) (end 79.84 102) (width 0.25) (layer "F.Cu") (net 3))
 (segment (start 95.05 69.35) (end 99.83 69.35) (width 0.25) (layer "F.Cu") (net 3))
 (segment (start 110.04 90.99) (end 111.76 92.71) (width 0.25) (layer "F.Cu") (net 3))
 (segment (start 71.12 71.12) (end 70.54 71.7) (width 0.25) (layer "F.Cu") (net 3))
 (segment (start 111.54 70.07) (end 111.54 68.6) (width 0.25) (layer "F.Cu") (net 3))
 (segment (start 81.64 94.34) (end 82.55 95.25) (width 0.25) (layer "F.Cu") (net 3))
 (segment (start 94.24 63.1) (end 94.24 68.54) (width 0.25) (layer "F.Cu") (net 3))
 (segment (start 94.24 58.16) (end 94.24 63.1) (width 0.25) (layer "F.Cu") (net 3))
 (segment (start 88.48 100) (end 81.529456 100) (width 0.25) (layer "F.Cu") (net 3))
 (segment (start 99.83 69.35) (end 101.6 71.12) (width 0.25) (layer "F.Cu") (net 3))
 (segment (start 81.28 71.12) (end 71.12 71.12) (width 0.25) (layer "F.Cu") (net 3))
 (segment (start 83.03 68.1) (end 84.28 69.35) (width 0.25) (layer "F.Cu") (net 3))
 (segment (start 97.3 55.1) (end 94.24 58.16) (width 0.25) (layer "F.Cu") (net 3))
 (segment (start 81.64 86.6) (end 81.64 71.48) (width 0.25) (layer "F.Cu") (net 3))
 (segment (start 84.28 69.35) (end 88.55 69.35) (width 0.25) (layer "F.Cu") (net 3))
 (segment (start 111.76 92.71) (end 113.03 92.71) (width 0.25) (layer "F.Cu") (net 3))
 (segment (start 94.24 68.54) (end 95.05 69.35) (width 0.25) (layer "F.Cu") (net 3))
 (segment (start 83.03 67.1) (end 83.03 69.37) (width 0.25) (layer "F.Cu") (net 3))
 (segment (start 110.49 71.12) (end 111.54 70.07) (width 0.25) (layer "F.Cu") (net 3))
 (via (at 82.55 95.25) (size 0.8) (drill 0.4) (layers "F.Cu" "B.Cu") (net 3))
 (segment (start 122.44 72.664728) (end 122.44 74) (width 0.25) (layer "B.Cu") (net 3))
 (segment (start 84.76 100) (end 88.48 100) (width 0.25) (layer "B.Cu") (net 3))
 (segment (start 120.895272 71.12) (end 122.44 72.664728) (width 0.25) (layer "B.Cu") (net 3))
 (segment (start 120.65 80.01) (end 111.125 80.01) (width 0.25) (layer "B.Cu") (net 3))
 (segment (start 110.04 81.095) (end 110.04 87) (width 0.25) (layer "B.Cu") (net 3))
 (segment (start 82.55 97.79) (end 84.76 100) (width 0.25) (layer "B.Cu") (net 3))
 (segment (start 113.03 71.12) (end 120.895272 71.12) (width 0.25) (layer "B.Cu") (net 3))
 (segment (start 111.125 80.01) (end 110.04 81.095) (width 0.25) (layer "B.Cu") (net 3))
 (segment (start 82.55 95.25) (end 82.55 97.79) (width 0.25) (layer "B.Cu") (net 3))
 (segment (start 111.54 68.6) (end 111.54 69.63) (width 0.25) (layer "B.Cu") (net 3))
 (segment (start 122.44 74) (end 122.44 78.22) (width 0.25) (layer "B.Cu") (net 3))
 (segment (start 111.54 69.63) (end 113.03 71.12) (width 0.25) (layer "B.Cu") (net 3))
 (segment (start 122.44 78.22) (end 120.65 80.01) (width 0.25) (layer "B.Cu") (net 3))
 (segment (start 109.22 72.39) (end 111.76 72.39) (width 0.25) (layer "F.Cu") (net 13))
 (segment (start 100.33 86.36) (end 100.33 80.01) (width 0.25) (layer "F.Cu") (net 13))
 (segment (start 101.6 78.74) (end 106.68 78.74) (width 0.25) (layer "F.Cu") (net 13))
 (segment (start 106.68 78.74) (end 107.95 77.47) (width 0.25) (layer "F.Cu") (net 13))
 (segment (start 100.33 80.01) (end 101.6 78.74) (width 0.25) (layer "F.Cu") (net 13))
 (segment (start 107.95 73.66) (end 109.22 72.39) (width 0.25) (layer "F.Cu") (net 13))
 (segment (start 101.27 87.3) (end 100.33 86.36) (width 0.25) (layer "F.Cu") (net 13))
 (segment (start 107.95 77.47) (end 107.95 73.66) (width 0.25) (layer "F.Cu") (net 13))
 (segment (start 103.72 87.3) (end 101.27 87.3) (width 0.25) (layer "F.Cu") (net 13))
 (segment (start 112.81 71.34) (end 112.81 68.6) (width 0.25) (layer "F.Cu") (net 13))
 (segment (start 111.76 72.39) (end 112.81 71.34) (width 0.25) (layer "F.Cu") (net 13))
 (segment (start 111.31 75.38) (end 111.31 87) (width 0.25) (layer "F.Cu") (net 5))
 (segment (start 119.9 74) (end 112.69 74) (width 0.25) (layer "F.Cu") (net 5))
 (segment (start 112.69 74) (end 111.31 75.38) (width 0.25) (layer "F.Cu") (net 5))
 (segment (start 107.5 87) (end 107.5 93.53) (width 0.25) (layer "B.Cu") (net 12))
 (segment (start 114.3 95.25) (end 116.11 97.06) (width 0.25) (layer "B.Cu") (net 12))
 (segment (start 109.22 95.25) (end 114.3 95.25) (width 0.25) (layer "B.Cu") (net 12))
 (segment (start 116.11 97.06) (end 116.11 104.4) (width 0.25) (layer "B.Cu") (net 12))
 (segment (start 107.5 93.53) (end 109.22 95.25) (width 0.25) (layer "B.Cu") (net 12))
 (segment (start 101.86 104.4) (end 112.3 104.4) (width 0.25) (layer "B.Cu") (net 4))
 (segment (start 99.46 102) (end 101.86 104.4) (width 0.25) (layer "B.Cu") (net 4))
 (segment (start 81.11 102) (end 99.46 102) (width 0.25) (layer "B.Cu") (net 4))
 (segment (start 78.74 95.25) (end 81.28 95.25) (width 0.25) (layer "B.Cu") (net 1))
 (segment (start 77.3 96.69) (end 78.74 95.25) (width 0.25) (layer "B.Cu") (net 1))
 (segment (start 77.3 102) (end 77.3 96.69) (width 0.25) (layer "B.Cu") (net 1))
 (segment (start 82.91 93.62) (end 82.91 86.6) (width 0.25) (layer "B.Cu") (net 1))
 (segment (start 81.28 95.25) (end 82.91 93.62) (width 0.25) (layer "B.Cu") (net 1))
 (segment (start 71.81 73.1) (end 71.81 75.62) (width 0.25) (layer "F.Cu") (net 11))
 (segment (start 71.81 75.62) (end 73.66 77.47) (width 0.25) (layer "F.Cu") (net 11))
 (segment (start 73.66 77.47) (end 77.47 77.47) (width 0.25) (layer "F.Cu") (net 11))
 (segment (start 79.1 79.1) (end 79.1 86.6) (width 0.25) (layer "F.Cu") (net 11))
 (segment (start 77.47 77.47) (end 79.1 79.1) (width 0.25) (layer "F.Cu") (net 11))
 (segment (start 68 71.7) (end 68 73.1) (width 0.25) (layer "B.Cu") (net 8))
 (segment (start 84.3 67.1) (end 84.3 68.1) (width 0.25) (layer "B.Cu") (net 8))
 (segment (start 82.55 69.85) (end 69.85 69.85) (width 0.25) (layer "B.Cu") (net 8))
 (segment (start 69.85 69.85) (end 68 71.7) (width 0.25) (layer "B.Cu") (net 8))
 (segment (start 84.3 68.1) (end 82.55 69.85) (width 0.25) (layer "B.Cu") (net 8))
 (segment (start 95.05 73.85) (end 88.55 73.85) (width 0.25) (layer "F.Cu") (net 9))
 (segment (start 95.05 73.85) (end 96.71 73.85) (width 0.25) (layer "F.Cu") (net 9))
 (segment (start 88.48 73.92) (end 88.55 73.85) (width 0.25) (layer "F.Cu") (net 9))
 (segment (start 88.48 82.22) (end 88.48 73.92) (width 0.25) (layer "F.Cu") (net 9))
 (segment (start 96.71 73.85) (end 98.68 75.82) (width 0.25) (layer "F.Cu") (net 9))
 (segment (start 98.68 75.82) (end 101.5 75.82) (width 0.25) (layer "F.Cu") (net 9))
 (segment (start 95.51 63.1) (end 95.51 65.78) (width 0.25) (layer "B.Cu") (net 7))
 (segment (start 95.51 65.78) (end 93.98 67.31) (width 0.25) (layer "B.Cu") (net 7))
 (segment (start 88.9 67.31) (end 86.36 64.77) (width 0.25) (layer "B.Cu") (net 7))
 (segment (start 86.36 64.77) (end 81.259728 64.77) (width 0.25) (layer "B.Cu") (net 7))
 (segment (start 93.98 67.31) (end 88.9 67.31) (width 0.25) (layer "B.Cu") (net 7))
 (segment (start 81.259728 64.77) (end 80.49 65.539728) (width 0.25) (layer "B.Cu") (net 7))
 (segment (start 80.49 65.539728) (end 80.49 67.1) (width 0.25) (layer "B.Cu") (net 7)))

